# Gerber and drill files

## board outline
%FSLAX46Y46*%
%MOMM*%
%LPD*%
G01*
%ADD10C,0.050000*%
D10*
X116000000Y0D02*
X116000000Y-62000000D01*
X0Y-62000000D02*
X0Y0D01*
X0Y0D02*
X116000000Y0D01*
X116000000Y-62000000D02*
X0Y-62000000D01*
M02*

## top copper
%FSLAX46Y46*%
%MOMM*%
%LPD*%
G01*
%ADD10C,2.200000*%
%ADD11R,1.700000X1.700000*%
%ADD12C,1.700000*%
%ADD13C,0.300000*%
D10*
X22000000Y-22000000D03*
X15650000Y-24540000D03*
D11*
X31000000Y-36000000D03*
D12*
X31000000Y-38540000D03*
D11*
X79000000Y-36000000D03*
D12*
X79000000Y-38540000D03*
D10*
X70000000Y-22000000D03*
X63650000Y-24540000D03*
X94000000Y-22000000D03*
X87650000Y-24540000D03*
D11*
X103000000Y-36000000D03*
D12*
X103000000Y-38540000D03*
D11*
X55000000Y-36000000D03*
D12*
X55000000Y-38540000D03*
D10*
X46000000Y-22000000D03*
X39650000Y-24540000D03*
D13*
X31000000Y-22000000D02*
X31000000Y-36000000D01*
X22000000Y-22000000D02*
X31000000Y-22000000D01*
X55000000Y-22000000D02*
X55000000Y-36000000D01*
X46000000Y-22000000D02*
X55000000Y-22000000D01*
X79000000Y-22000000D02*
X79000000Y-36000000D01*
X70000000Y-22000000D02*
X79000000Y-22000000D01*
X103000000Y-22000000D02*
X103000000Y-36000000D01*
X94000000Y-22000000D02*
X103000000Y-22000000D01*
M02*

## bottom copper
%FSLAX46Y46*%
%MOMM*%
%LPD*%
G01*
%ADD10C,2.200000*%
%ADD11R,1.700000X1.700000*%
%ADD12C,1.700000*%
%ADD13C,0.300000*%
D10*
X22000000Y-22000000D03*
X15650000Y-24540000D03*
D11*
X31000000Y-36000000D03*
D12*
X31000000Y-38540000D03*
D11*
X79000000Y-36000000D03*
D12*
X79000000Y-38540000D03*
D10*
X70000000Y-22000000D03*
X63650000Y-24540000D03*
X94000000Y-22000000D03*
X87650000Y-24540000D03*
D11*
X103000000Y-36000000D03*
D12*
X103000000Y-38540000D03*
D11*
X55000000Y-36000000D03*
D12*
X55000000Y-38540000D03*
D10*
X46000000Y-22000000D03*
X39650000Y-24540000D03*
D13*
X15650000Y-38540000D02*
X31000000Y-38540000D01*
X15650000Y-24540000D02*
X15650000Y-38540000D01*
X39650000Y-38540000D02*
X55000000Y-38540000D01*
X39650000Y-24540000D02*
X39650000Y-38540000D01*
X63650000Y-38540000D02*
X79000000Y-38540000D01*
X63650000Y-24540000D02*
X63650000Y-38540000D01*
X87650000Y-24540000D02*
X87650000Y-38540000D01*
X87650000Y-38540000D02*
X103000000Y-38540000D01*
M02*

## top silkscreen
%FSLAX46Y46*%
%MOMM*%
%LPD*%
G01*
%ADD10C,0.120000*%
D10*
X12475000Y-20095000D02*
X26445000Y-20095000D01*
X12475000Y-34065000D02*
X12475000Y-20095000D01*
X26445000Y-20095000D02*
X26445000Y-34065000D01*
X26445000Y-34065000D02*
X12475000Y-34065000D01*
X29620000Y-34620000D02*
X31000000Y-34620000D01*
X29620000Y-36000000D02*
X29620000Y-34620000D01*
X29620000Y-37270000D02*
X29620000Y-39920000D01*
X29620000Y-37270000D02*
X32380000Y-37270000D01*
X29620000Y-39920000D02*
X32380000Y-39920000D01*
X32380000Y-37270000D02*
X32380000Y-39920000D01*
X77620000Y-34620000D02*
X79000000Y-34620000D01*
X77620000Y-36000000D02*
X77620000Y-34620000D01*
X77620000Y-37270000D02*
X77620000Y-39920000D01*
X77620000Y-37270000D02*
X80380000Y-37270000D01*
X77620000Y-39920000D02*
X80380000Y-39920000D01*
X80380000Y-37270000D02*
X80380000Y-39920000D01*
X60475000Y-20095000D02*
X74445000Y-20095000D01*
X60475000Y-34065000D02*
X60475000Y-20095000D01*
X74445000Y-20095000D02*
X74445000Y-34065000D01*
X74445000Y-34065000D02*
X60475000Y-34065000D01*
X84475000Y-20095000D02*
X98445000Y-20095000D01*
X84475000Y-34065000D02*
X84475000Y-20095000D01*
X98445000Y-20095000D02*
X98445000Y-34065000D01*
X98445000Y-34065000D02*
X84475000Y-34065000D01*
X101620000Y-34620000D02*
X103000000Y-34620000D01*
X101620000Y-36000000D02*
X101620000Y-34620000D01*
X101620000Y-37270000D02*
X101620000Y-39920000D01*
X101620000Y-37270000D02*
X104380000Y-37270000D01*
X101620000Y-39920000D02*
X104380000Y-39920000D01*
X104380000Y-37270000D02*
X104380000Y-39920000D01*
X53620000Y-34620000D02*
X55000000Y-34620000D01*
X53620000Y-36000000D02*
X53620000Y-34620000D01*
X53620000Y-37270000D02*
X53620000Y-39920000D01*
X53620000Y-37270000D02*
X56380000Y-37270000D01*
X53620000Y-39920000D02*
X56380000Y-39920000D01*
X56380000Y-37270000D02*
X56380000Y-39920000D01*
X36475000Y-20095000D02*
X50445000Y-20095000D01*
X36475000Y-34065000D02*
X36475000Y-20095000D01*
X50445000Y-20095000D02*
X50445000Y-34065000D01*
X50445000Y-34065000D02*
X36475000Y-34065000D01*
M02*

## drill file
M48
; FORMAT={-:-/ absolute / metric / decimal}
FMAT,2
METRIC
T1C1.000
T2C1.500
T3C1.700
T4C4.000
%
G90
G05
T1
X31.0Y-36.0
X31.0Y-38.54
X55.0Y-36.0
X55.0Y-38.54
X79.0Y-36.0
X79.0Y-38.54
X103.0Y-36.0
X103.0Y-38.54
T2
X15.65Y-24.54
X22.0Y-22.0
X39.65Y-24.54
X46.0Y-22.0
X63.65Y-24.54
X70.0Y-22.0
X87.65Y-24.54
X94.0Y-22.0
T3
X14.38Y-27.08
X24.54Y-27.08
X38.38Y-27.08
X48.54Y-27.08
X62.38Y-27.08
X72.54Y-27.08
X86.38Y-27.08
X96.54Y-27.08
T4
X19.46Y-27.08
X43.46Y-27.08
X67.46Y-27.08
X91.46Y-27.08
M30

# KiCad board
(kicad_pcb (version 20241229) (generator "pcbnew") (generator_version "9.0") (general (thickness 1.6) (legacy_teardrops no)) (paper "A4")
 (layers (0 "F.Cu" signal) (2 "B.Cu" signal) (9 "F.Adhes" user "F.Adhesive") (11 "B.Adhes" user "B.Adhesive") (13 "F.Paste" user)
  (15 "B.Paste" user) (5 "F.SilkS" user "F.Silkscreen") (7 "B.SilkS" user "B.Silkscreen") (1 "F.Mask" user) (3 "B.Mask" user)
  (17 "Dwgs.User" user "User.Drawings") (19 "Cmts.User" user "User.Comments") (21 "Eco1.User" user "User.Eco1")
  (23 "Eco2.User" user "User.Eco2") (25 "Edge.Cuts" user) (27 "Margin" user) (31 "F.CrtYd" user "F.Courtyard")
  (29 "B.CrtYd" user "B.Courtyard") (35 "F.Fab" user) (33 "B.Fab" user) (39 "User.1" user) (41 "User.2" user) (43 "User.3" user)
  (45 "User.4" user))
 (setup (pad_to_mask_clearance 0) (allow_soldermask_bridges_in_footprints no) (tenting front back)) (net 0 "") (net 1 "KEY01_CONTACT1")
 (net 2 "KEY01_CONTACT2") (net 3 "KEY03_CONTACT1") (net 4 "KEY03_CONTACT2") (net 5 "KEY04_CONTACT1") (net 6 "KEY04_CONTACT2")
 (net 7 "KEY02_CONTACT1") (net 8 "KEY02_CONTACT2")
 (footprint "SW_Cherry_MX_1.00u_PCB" (layer "F.Cu") (at 22 22)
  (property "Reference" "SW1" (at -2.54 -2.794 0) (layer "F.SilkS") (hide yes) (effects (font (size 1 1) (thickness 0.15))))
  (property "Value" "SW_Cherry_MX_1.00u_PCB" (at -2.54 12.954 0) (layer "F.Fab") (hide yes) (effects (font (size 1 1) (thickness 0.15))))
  (fp_line (start -9.525 -1.905) (end 4.445 -1.905) (stroke (width 0.12) (type solid)) (layer "F.SilkS"))
  (fp_line (start -9.525 12.065) (end -9.525 -1.905) (stroke (width 0.12) (type solid)) (layer "F.SilkS"))
  (fp_line (start 4.445 -1.905) (end 4.445 12.065) (stroke (width 0.12) (type solid)) (layer "F.SilkS"))
  (fp_line (start 4.445 12.065) (end -9.525 12.065) (stroke (width 0.12) (type solid)) (layer "F.SilkS"))
  (pad "" np_thru_hole circle (at -7.62 5.08) (size 1.7 1.7) (drill 1.7) (layers "*.Cu" "*.Mask"))
  (pad "" np_thru_hole circle (at -2.54 5.08) (size 4 4) (drill 4) (layers "*.Cu" "*.Mask"))
  (pad "" np_thru_hole circle (at 2.54 5.08) (size 1.7 1.7) (drill 1.7) (layers "*.Cu" "*.Mask"))
  (pad "1" thru_hole circle (at 0 0) (size 2.2 2.2) (drill 1.5) (layers "*.Cu" "*.Mask") (remove_unused_layers no) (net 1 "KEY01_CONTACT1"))
  (pad "2" thru_hole circle (at -6.35 2.54) (size 2.2 2.2) (drill 1.5) (layers "*.Cu" "*.Mask") (remove_unused_layers no)
   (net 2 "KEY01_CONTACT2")))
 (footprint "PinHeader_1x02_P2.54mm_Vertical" (layer "F.Cu") (at 31 36)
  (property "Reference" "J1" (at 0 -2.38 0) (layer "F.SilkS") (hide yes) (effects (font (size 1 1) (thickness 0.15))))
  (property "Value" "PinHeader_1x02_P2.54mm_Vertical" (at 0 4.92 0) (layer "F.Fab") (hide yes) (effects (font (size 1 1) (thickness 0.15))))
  (fp_line (start -1.38 -1.38) (end 0 -1.38) (stroke (width 0.12) (type solid)) (layer "F.SilkS"))
  (fp_line (start -1.38 0) (end -1.38 -1.38) (stroke (width 0.12) (type solid)) (layer "F.SilkS"))
  (fp_line (start -1.38 1.27) (end -1.38 3.92) (stroke (width 0.12) (type solid)) (layer "F.SilkS"))
  (fp_line (start -1.38 1.27) (end 1.38 1.27) (stroke (width 0.12) (type solid)) (layer "F.SilkS"))
  (fp_line (start -1.38 3.92) (end 1.38 3.92) (stroke (width 0.12) (type solid)) (layer "F.SilkS"))
  (fp_line (start 1.38 1.27) (end 1.38 3.92) (stroke (width 0.12) (type solid)) (layer "F.SilkS"))
  (pad "1" thru_hole rect (at 0 0) (size 1.7 1.7) (drill 1) (layers "*.Cu" "*.Mask") (remove_unused_layers no) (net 1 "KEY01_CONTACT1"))
  (pad "2" thru_hole circle (at 0 2.54) (size 1.7 1.7) (drill 1) (layers "*.Cu" "*.Mask") (remove_unused_layers no) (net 2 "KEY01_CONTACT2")))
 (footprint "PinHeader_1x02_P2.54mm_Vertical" (layer "F.Cu") (at 79 36)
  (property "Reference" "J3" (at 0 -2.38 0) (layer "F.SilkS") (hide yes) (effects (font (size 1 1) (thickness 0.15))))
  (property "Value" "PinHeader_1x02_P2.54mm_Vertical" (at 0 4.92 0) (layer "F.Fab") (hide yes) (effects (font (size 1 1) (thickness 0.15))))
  (fp_line (start -1.38 -1.38) (end 0 -1.38) (stroke (width 0.12) (type solid)) (layer "F.SilkS"))
  (fp_line (start -1.38 0) (end -1.38 -1.38) (stroke (width 0.12) (type solid)) (layer "F.SilkS"))
  (fp_line (start -1.38 1.27) (end -1.38 3.92) (stroke (width 0.12) (type solid)) (layer "F.SilkS"))
  (fp_line (start -1.38 1.27) (end 1.38 1.27) (stroke (width 0.12) (type solid)) (layer "F.SilkS"))
  (fp_line (start -1.38 3.92) (end 1.38 3.92) (stroke (width 0.12) (type solid)) (layer "F.SilkS"))
  (fp_line (start 1.38 1.27) (end 1.38 3.92) (stroke (width 0.12) (type solid)) (layer "F.SilkS"))
  (pad "1" thru_hole rect (at 0 0) (size 1.7 1.7) (drill 1) (layers "*.Cu" "*.Mask") (remove_unused_layers no) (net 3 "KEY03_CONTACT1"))
  (pad "2" thru_hole circle (at 0 2.54) (size 1.7 1.7) (drill 1) (layers "*.Cu" "*.Mask") (remove_unused_layers no) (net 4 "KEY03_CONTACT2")))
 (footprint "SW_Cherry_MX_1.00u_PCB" (layer "F.Cu") (at 70 22)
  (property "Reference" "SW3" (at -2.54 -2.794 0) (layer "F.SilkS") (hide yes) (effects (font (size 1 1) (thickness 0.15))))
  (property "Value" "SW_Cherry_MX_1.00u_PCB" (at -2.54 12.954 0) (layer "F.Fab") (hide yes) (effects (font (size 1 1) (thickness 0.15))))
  (fp_line (start -9.525 -1.905) (end 4.445 -1.905) (stroke (width 0.12) (type solid)) (layer "F.SilkS"))
  (fp_line (start -9.525 12.065) (end -9.525 -1.905) (stroke (width 0.12) (type solid)) (layer "F.SilkS"))
  (fp_line (start 4.445 -1.905) (end 4.445 12.065) (stroke (width 0.12) (type solid)) (layer "F.SilkS"))
  (fp_line (start 4.445 12.065) (end -9.525 12.065) (stroke (width 0.12) (type solid)) (layer "F.SilkS"))
  (pad "" np_thru_hole circle (at -7.62 5.08) (size 1.7 1.7) (drill 1.7) (layers "*.Cu" "*.Mask"))
  (pad "" np_thru_hole circle (at -2.54 5.08) (size 4 4) (drill 4) (layers "*.Cu" "*.Mask"))
  (pad "" np_thru_hole circle (at 2.54 5.08) (size 1.7 1.7) (drill 1.7) (layers "*.Cu" "*.Mask"))
  (pad "1" thru_hole circle (at 0 0) (size 2.2 2.2) (drill 1.5) (layers "*.Cu" "*.Mask") (remove_unused_layers no) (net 3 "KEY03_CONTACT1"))
  (pad "2" thru_hole circle (at -6.35 2.54) (size 2.2 2.2) (drill 1.5) (layers "*.Cu" "*.Mask") (remove_unused_layers no)
   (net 4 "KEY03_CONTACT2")))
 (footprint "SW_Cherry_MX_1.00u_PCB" (layer "F.Cu") (at 94 22)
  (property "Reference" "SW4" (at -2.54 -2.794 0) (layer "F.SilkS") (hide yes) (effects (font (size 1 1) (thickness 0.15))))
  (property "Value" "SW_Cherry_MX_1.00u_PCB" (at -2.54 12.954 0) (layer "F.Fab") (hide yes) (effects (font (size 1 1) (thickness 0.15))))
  (fp_line (start -9.525 -1.905) (end 4.445 -1.905) (stroke (width 0.12) (type solid)) (layer "F.SilkS"))
  (fp_line (start -9.525 12.065) (end -9.525 -1.905) (stroke (width 0.12) (type solid)) (layer "F.SilkS"))
  (fp_line (start 4.445 -1.905) (end 4.445 12.065) (stroke (width 0.12) (type solid)) (layer "F.SilkS"))
  (fp_line (start 4.445 12.065) (end -9.525 12.065) (stroke (width 0.12) (type solid)) (layer "F.SilkS"))
  (pad "" np_thru_hole circle (at -7.62 5.08) (size 1.7 1.7) (drill 1.7) (layers "*.Cu" "*.Mask"))
  (pad "" np_thru_hole circle (at -2.54 5.08) (size 4 4) (drill 4) (layers "*.Cu" "*.Mask"))
  (pad "" np_thru_hole circle (at 2.54 5.08) (size 1.7 1.7) (drill 1.7) (layers "*.Cu" "*.Mask"))
  (pad "1" thru_hole circle (at 0 0) (size 2.2 2.2) (drill 1.5) (layers "*.Cu" "*.Mask") (remove_unused_layers no) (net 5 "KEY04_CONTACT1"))
  (pad "2" thru_hole circle (at -6.35 2.54) (size 2.2 2.2) (drill 1.5) (layers "*.Cu" "*.Mask") (remove_unused_layers no)
   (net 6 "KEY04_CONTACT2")))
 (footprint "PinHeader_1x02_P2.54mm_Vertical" (layer "F.Cu") (at 103 36)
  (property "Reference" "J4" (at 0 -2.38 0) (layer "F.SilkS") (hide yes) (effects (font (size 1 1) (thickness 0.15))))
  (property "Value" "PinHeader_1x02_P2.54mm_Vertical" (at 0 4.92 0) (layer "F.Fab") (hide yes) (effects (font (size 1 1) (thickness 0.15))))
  (fp_line (start -1.38 -1.38) (end 0 -1.38) (stroke (width 0.12) (type solid)) (layer "F.SilkS"))
  (fp_line (start -1.38 0) (end -1.38 -1.38) (stroke (width 0.12) (type solid)) (layer "F.SilkS"))
  (fp_line (start -1.38 1.27) (end -1.38 3.92) (stroke (width 0.12) (type solid)) (layer "F.SilkS"))
  (fp_line (start -1.38 1.27) (end 1.38 1.27) (stroke (width 0.12) (type solid)) (layer "F.SilkS"))
  (fp_line (start -1.38 3.92) (end 1.38 3.92) (stroke (width 0.12) (type solid)) (layer "F.SilkS"))
  (fp_line (start 1.38 1.27) (end 1.38 3.92) (stroke (width 0.12) (type solid)) (layer "F.SilkS"))
  (pad "1" thru_hole rect (at 0 0) (size 1.7 1.7) (drill 1) (layers "*.Cu" "*.Mask") (remove_unused_layers no) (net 5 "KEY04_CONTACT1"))
  (pad "2" thru_hole circle (at 0 2.54) (size 1.7 1.7) (drill 1) (layers "*.Cu" "*.Mask") (remove_unused_layers no) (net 6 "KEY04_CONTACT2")))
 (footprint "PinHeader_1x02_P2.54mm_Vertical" (layer "F.Cu") (at 55 36)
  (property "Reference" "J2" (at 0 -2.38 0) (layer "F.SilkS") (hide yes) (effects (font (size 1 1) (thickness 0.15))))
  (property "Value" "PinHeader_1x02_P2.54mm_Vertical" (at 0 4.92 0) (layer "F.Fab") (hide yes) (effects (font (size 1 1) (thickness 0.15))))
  (fp_line (start -1.38 -1.38) (end 0 -1.38) (stroke (width 0.12) (type solid)) (layer "F.SilkS"))
  (fp_line (start -1.38 0) (end -1.38 -1.38) (stroke (width 0.12) (type solid)) (layer "F.SilkS"))
  (fp_line (start -1.38 1.27) (end -1.38 3.92) (stroke (width 0.12) (type solid)) (layer "F.SilkS"))
  (fp_line (start -1.38 1.27) (end 1.38 1.27) (stroke (width 0.12) (type solid)) (layer "F.SilkS"))
  (fp_line (start -1.38 3.92) (end 1.38 3.92) (stroke (width 0.12) (type solid)) (layer "F.SilkS"))
  (fp_line (start 1.38 1.27) (end 1.38 3.92) (stroke (width 0.12) (type solid)) (layer "F.SilkS"))
  (pad "1" thru_hole rect (at 0 0) (size 1.7 1.7) (drill 1) (layers "*.Cu" "*.Mask") (remove_unused_layers no) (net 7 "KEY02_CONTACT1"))
  (pad "2" thru_hole circle (at 0 2.54) (size 1.7 1.7) (drill 1) (layers "*.Cu" "*.Mask") (remove_unused_layers no) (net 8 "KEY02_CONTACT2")))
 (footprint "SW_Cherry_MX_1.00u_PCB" (layer "F.Cu") (at 46 22)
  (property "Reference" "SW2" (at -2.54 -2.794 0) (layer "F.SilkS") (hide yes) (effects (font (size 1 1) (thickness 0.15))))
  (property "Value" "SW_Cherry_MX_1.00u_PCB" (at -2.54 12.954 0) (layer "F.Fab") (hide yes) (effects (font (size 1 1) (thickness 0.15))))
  (fp_line (start -9.525 -1.905) (end 4.445 -1.905) (stroke (width 0.12) (type solid)) (layer "F.SilkS"))
  (fp_line (start -9.525 12.065) (end -9.525 -1.905) (stroke (width 0.12) (type solid)) (layer "F.SilkS"))
  (fp_line (start 4.445 -1.905) (end 4.445 12.065) (stroke (width 0.12) (type solid)) (layer "F.SilkS"))
  (fp_line (start 4.445 12.065) (end -9.525 12.065) (stroke (width 0.12) (type solid)) (layer "F.SilkS"))
  (pad "" np_thru_hole circle (at -7.62 5.08) (size 1.7 1.7) (drill 1.7) (layers "*.Cu" "*.Mask"))
  (pad "" np_thru_hole circle (at -2.54 5.08) (size 4 4) (drill 4) (layers "*.Cu" "*.Mask"))
  (pad "" np_thru_hole circle (at 2.54 5.08) (size 1.7 1.7) (drill 1.7) (layers "*.Cu" "*.Mask"))
  (pad "1" thru_hole circle (at 0 0) (size 2.2 2.2) (drill 1.5) (layers "*.Cu" "*.Mask") (remove_unused_layers no) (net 7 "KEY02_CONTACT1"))
  (pad "2" thru_hole circle (at -6.35 2.54) (size 2.2 2.2) (drill 1.5) (layers "*.Cu" "*.Mask") (remove_unused_layers no)
   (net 8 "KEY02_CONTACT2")))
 (gr_line (start 116 0) (end 116 62) (stroke (width 0.05) (type default)) (layer "Edge.Cuts"))
 (gr_line (start 0 62) (end 0 0) (stroke (width 0.05) (type default)) (layer "Edge.Cuts"))
 (gr_line (start 0 0) (end 116 0) (stroke (width 0.05) (type default)) (layer "Edge.Cuts"))
 (gr_line (start 116 62) (end 0 62) (stroke (width 0.05) (type default)) (layer "Edge.Cuts"))
 (segment (start 31 22) (end 31 36) (width 0.3) (layer "F.Cu") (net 1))
 (segment (start 22 22) (end 31 22) (width 0.3) (layer "F.Cu") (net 1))
 (segment (start 15.65 38.54) (end 31 38.54) (width 0.3) (layer "B.Cu") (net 2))
 (segment (start 15.65 24.54) (end 15.65 38.54) (width 0.3) (layer "B.Cu") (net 2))
 (segment (start 55 22) (end 55 36) (width 0.3) (layer "F.Cu") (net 7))
 (segment (start 46 22) (end 55 22) (width 0.3) (layer "F.Cu") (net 7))
 (segment (start 39.65 38.54) (end 55 38.54) (width 0.3) (layer "B.Cu") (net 8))
 (segment (start 39.65 24.54) (end 39.65 38.54) (width 0.3) (layer "B.Cu") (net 8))
 (segment (start 79 22) (end 79 36) (width 0.3) (layer "F.Cu") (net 3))
 (segment (start 70 22) (end 79 22) (width 0.3) (layer "F.Cu") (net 3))
 (segment (start 63.65 38.54) (end 79 38.54) (width 0.3) (layer "B.Cu") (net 4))
 (segment (start 63.65 24.54) (end 63.65 38.54) (width 0.3) (layer "B.Cu") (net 4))
 (segment (start 103 22) (end 103 36) (width 0.3) (layer "F.Cu") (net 5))
 (segment (start 94 22) (end 103 22) (width 0.3) (layer "F.Cu") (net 5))
 (segment (start 87.65 24.54) (end 87.65 38.54) (width 0.3) (layer "B.Cu") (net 6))
 (segment (start 87.65 38.54) (end 103 38.54) (width 0.3) (layer "B.Cu") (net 6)))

